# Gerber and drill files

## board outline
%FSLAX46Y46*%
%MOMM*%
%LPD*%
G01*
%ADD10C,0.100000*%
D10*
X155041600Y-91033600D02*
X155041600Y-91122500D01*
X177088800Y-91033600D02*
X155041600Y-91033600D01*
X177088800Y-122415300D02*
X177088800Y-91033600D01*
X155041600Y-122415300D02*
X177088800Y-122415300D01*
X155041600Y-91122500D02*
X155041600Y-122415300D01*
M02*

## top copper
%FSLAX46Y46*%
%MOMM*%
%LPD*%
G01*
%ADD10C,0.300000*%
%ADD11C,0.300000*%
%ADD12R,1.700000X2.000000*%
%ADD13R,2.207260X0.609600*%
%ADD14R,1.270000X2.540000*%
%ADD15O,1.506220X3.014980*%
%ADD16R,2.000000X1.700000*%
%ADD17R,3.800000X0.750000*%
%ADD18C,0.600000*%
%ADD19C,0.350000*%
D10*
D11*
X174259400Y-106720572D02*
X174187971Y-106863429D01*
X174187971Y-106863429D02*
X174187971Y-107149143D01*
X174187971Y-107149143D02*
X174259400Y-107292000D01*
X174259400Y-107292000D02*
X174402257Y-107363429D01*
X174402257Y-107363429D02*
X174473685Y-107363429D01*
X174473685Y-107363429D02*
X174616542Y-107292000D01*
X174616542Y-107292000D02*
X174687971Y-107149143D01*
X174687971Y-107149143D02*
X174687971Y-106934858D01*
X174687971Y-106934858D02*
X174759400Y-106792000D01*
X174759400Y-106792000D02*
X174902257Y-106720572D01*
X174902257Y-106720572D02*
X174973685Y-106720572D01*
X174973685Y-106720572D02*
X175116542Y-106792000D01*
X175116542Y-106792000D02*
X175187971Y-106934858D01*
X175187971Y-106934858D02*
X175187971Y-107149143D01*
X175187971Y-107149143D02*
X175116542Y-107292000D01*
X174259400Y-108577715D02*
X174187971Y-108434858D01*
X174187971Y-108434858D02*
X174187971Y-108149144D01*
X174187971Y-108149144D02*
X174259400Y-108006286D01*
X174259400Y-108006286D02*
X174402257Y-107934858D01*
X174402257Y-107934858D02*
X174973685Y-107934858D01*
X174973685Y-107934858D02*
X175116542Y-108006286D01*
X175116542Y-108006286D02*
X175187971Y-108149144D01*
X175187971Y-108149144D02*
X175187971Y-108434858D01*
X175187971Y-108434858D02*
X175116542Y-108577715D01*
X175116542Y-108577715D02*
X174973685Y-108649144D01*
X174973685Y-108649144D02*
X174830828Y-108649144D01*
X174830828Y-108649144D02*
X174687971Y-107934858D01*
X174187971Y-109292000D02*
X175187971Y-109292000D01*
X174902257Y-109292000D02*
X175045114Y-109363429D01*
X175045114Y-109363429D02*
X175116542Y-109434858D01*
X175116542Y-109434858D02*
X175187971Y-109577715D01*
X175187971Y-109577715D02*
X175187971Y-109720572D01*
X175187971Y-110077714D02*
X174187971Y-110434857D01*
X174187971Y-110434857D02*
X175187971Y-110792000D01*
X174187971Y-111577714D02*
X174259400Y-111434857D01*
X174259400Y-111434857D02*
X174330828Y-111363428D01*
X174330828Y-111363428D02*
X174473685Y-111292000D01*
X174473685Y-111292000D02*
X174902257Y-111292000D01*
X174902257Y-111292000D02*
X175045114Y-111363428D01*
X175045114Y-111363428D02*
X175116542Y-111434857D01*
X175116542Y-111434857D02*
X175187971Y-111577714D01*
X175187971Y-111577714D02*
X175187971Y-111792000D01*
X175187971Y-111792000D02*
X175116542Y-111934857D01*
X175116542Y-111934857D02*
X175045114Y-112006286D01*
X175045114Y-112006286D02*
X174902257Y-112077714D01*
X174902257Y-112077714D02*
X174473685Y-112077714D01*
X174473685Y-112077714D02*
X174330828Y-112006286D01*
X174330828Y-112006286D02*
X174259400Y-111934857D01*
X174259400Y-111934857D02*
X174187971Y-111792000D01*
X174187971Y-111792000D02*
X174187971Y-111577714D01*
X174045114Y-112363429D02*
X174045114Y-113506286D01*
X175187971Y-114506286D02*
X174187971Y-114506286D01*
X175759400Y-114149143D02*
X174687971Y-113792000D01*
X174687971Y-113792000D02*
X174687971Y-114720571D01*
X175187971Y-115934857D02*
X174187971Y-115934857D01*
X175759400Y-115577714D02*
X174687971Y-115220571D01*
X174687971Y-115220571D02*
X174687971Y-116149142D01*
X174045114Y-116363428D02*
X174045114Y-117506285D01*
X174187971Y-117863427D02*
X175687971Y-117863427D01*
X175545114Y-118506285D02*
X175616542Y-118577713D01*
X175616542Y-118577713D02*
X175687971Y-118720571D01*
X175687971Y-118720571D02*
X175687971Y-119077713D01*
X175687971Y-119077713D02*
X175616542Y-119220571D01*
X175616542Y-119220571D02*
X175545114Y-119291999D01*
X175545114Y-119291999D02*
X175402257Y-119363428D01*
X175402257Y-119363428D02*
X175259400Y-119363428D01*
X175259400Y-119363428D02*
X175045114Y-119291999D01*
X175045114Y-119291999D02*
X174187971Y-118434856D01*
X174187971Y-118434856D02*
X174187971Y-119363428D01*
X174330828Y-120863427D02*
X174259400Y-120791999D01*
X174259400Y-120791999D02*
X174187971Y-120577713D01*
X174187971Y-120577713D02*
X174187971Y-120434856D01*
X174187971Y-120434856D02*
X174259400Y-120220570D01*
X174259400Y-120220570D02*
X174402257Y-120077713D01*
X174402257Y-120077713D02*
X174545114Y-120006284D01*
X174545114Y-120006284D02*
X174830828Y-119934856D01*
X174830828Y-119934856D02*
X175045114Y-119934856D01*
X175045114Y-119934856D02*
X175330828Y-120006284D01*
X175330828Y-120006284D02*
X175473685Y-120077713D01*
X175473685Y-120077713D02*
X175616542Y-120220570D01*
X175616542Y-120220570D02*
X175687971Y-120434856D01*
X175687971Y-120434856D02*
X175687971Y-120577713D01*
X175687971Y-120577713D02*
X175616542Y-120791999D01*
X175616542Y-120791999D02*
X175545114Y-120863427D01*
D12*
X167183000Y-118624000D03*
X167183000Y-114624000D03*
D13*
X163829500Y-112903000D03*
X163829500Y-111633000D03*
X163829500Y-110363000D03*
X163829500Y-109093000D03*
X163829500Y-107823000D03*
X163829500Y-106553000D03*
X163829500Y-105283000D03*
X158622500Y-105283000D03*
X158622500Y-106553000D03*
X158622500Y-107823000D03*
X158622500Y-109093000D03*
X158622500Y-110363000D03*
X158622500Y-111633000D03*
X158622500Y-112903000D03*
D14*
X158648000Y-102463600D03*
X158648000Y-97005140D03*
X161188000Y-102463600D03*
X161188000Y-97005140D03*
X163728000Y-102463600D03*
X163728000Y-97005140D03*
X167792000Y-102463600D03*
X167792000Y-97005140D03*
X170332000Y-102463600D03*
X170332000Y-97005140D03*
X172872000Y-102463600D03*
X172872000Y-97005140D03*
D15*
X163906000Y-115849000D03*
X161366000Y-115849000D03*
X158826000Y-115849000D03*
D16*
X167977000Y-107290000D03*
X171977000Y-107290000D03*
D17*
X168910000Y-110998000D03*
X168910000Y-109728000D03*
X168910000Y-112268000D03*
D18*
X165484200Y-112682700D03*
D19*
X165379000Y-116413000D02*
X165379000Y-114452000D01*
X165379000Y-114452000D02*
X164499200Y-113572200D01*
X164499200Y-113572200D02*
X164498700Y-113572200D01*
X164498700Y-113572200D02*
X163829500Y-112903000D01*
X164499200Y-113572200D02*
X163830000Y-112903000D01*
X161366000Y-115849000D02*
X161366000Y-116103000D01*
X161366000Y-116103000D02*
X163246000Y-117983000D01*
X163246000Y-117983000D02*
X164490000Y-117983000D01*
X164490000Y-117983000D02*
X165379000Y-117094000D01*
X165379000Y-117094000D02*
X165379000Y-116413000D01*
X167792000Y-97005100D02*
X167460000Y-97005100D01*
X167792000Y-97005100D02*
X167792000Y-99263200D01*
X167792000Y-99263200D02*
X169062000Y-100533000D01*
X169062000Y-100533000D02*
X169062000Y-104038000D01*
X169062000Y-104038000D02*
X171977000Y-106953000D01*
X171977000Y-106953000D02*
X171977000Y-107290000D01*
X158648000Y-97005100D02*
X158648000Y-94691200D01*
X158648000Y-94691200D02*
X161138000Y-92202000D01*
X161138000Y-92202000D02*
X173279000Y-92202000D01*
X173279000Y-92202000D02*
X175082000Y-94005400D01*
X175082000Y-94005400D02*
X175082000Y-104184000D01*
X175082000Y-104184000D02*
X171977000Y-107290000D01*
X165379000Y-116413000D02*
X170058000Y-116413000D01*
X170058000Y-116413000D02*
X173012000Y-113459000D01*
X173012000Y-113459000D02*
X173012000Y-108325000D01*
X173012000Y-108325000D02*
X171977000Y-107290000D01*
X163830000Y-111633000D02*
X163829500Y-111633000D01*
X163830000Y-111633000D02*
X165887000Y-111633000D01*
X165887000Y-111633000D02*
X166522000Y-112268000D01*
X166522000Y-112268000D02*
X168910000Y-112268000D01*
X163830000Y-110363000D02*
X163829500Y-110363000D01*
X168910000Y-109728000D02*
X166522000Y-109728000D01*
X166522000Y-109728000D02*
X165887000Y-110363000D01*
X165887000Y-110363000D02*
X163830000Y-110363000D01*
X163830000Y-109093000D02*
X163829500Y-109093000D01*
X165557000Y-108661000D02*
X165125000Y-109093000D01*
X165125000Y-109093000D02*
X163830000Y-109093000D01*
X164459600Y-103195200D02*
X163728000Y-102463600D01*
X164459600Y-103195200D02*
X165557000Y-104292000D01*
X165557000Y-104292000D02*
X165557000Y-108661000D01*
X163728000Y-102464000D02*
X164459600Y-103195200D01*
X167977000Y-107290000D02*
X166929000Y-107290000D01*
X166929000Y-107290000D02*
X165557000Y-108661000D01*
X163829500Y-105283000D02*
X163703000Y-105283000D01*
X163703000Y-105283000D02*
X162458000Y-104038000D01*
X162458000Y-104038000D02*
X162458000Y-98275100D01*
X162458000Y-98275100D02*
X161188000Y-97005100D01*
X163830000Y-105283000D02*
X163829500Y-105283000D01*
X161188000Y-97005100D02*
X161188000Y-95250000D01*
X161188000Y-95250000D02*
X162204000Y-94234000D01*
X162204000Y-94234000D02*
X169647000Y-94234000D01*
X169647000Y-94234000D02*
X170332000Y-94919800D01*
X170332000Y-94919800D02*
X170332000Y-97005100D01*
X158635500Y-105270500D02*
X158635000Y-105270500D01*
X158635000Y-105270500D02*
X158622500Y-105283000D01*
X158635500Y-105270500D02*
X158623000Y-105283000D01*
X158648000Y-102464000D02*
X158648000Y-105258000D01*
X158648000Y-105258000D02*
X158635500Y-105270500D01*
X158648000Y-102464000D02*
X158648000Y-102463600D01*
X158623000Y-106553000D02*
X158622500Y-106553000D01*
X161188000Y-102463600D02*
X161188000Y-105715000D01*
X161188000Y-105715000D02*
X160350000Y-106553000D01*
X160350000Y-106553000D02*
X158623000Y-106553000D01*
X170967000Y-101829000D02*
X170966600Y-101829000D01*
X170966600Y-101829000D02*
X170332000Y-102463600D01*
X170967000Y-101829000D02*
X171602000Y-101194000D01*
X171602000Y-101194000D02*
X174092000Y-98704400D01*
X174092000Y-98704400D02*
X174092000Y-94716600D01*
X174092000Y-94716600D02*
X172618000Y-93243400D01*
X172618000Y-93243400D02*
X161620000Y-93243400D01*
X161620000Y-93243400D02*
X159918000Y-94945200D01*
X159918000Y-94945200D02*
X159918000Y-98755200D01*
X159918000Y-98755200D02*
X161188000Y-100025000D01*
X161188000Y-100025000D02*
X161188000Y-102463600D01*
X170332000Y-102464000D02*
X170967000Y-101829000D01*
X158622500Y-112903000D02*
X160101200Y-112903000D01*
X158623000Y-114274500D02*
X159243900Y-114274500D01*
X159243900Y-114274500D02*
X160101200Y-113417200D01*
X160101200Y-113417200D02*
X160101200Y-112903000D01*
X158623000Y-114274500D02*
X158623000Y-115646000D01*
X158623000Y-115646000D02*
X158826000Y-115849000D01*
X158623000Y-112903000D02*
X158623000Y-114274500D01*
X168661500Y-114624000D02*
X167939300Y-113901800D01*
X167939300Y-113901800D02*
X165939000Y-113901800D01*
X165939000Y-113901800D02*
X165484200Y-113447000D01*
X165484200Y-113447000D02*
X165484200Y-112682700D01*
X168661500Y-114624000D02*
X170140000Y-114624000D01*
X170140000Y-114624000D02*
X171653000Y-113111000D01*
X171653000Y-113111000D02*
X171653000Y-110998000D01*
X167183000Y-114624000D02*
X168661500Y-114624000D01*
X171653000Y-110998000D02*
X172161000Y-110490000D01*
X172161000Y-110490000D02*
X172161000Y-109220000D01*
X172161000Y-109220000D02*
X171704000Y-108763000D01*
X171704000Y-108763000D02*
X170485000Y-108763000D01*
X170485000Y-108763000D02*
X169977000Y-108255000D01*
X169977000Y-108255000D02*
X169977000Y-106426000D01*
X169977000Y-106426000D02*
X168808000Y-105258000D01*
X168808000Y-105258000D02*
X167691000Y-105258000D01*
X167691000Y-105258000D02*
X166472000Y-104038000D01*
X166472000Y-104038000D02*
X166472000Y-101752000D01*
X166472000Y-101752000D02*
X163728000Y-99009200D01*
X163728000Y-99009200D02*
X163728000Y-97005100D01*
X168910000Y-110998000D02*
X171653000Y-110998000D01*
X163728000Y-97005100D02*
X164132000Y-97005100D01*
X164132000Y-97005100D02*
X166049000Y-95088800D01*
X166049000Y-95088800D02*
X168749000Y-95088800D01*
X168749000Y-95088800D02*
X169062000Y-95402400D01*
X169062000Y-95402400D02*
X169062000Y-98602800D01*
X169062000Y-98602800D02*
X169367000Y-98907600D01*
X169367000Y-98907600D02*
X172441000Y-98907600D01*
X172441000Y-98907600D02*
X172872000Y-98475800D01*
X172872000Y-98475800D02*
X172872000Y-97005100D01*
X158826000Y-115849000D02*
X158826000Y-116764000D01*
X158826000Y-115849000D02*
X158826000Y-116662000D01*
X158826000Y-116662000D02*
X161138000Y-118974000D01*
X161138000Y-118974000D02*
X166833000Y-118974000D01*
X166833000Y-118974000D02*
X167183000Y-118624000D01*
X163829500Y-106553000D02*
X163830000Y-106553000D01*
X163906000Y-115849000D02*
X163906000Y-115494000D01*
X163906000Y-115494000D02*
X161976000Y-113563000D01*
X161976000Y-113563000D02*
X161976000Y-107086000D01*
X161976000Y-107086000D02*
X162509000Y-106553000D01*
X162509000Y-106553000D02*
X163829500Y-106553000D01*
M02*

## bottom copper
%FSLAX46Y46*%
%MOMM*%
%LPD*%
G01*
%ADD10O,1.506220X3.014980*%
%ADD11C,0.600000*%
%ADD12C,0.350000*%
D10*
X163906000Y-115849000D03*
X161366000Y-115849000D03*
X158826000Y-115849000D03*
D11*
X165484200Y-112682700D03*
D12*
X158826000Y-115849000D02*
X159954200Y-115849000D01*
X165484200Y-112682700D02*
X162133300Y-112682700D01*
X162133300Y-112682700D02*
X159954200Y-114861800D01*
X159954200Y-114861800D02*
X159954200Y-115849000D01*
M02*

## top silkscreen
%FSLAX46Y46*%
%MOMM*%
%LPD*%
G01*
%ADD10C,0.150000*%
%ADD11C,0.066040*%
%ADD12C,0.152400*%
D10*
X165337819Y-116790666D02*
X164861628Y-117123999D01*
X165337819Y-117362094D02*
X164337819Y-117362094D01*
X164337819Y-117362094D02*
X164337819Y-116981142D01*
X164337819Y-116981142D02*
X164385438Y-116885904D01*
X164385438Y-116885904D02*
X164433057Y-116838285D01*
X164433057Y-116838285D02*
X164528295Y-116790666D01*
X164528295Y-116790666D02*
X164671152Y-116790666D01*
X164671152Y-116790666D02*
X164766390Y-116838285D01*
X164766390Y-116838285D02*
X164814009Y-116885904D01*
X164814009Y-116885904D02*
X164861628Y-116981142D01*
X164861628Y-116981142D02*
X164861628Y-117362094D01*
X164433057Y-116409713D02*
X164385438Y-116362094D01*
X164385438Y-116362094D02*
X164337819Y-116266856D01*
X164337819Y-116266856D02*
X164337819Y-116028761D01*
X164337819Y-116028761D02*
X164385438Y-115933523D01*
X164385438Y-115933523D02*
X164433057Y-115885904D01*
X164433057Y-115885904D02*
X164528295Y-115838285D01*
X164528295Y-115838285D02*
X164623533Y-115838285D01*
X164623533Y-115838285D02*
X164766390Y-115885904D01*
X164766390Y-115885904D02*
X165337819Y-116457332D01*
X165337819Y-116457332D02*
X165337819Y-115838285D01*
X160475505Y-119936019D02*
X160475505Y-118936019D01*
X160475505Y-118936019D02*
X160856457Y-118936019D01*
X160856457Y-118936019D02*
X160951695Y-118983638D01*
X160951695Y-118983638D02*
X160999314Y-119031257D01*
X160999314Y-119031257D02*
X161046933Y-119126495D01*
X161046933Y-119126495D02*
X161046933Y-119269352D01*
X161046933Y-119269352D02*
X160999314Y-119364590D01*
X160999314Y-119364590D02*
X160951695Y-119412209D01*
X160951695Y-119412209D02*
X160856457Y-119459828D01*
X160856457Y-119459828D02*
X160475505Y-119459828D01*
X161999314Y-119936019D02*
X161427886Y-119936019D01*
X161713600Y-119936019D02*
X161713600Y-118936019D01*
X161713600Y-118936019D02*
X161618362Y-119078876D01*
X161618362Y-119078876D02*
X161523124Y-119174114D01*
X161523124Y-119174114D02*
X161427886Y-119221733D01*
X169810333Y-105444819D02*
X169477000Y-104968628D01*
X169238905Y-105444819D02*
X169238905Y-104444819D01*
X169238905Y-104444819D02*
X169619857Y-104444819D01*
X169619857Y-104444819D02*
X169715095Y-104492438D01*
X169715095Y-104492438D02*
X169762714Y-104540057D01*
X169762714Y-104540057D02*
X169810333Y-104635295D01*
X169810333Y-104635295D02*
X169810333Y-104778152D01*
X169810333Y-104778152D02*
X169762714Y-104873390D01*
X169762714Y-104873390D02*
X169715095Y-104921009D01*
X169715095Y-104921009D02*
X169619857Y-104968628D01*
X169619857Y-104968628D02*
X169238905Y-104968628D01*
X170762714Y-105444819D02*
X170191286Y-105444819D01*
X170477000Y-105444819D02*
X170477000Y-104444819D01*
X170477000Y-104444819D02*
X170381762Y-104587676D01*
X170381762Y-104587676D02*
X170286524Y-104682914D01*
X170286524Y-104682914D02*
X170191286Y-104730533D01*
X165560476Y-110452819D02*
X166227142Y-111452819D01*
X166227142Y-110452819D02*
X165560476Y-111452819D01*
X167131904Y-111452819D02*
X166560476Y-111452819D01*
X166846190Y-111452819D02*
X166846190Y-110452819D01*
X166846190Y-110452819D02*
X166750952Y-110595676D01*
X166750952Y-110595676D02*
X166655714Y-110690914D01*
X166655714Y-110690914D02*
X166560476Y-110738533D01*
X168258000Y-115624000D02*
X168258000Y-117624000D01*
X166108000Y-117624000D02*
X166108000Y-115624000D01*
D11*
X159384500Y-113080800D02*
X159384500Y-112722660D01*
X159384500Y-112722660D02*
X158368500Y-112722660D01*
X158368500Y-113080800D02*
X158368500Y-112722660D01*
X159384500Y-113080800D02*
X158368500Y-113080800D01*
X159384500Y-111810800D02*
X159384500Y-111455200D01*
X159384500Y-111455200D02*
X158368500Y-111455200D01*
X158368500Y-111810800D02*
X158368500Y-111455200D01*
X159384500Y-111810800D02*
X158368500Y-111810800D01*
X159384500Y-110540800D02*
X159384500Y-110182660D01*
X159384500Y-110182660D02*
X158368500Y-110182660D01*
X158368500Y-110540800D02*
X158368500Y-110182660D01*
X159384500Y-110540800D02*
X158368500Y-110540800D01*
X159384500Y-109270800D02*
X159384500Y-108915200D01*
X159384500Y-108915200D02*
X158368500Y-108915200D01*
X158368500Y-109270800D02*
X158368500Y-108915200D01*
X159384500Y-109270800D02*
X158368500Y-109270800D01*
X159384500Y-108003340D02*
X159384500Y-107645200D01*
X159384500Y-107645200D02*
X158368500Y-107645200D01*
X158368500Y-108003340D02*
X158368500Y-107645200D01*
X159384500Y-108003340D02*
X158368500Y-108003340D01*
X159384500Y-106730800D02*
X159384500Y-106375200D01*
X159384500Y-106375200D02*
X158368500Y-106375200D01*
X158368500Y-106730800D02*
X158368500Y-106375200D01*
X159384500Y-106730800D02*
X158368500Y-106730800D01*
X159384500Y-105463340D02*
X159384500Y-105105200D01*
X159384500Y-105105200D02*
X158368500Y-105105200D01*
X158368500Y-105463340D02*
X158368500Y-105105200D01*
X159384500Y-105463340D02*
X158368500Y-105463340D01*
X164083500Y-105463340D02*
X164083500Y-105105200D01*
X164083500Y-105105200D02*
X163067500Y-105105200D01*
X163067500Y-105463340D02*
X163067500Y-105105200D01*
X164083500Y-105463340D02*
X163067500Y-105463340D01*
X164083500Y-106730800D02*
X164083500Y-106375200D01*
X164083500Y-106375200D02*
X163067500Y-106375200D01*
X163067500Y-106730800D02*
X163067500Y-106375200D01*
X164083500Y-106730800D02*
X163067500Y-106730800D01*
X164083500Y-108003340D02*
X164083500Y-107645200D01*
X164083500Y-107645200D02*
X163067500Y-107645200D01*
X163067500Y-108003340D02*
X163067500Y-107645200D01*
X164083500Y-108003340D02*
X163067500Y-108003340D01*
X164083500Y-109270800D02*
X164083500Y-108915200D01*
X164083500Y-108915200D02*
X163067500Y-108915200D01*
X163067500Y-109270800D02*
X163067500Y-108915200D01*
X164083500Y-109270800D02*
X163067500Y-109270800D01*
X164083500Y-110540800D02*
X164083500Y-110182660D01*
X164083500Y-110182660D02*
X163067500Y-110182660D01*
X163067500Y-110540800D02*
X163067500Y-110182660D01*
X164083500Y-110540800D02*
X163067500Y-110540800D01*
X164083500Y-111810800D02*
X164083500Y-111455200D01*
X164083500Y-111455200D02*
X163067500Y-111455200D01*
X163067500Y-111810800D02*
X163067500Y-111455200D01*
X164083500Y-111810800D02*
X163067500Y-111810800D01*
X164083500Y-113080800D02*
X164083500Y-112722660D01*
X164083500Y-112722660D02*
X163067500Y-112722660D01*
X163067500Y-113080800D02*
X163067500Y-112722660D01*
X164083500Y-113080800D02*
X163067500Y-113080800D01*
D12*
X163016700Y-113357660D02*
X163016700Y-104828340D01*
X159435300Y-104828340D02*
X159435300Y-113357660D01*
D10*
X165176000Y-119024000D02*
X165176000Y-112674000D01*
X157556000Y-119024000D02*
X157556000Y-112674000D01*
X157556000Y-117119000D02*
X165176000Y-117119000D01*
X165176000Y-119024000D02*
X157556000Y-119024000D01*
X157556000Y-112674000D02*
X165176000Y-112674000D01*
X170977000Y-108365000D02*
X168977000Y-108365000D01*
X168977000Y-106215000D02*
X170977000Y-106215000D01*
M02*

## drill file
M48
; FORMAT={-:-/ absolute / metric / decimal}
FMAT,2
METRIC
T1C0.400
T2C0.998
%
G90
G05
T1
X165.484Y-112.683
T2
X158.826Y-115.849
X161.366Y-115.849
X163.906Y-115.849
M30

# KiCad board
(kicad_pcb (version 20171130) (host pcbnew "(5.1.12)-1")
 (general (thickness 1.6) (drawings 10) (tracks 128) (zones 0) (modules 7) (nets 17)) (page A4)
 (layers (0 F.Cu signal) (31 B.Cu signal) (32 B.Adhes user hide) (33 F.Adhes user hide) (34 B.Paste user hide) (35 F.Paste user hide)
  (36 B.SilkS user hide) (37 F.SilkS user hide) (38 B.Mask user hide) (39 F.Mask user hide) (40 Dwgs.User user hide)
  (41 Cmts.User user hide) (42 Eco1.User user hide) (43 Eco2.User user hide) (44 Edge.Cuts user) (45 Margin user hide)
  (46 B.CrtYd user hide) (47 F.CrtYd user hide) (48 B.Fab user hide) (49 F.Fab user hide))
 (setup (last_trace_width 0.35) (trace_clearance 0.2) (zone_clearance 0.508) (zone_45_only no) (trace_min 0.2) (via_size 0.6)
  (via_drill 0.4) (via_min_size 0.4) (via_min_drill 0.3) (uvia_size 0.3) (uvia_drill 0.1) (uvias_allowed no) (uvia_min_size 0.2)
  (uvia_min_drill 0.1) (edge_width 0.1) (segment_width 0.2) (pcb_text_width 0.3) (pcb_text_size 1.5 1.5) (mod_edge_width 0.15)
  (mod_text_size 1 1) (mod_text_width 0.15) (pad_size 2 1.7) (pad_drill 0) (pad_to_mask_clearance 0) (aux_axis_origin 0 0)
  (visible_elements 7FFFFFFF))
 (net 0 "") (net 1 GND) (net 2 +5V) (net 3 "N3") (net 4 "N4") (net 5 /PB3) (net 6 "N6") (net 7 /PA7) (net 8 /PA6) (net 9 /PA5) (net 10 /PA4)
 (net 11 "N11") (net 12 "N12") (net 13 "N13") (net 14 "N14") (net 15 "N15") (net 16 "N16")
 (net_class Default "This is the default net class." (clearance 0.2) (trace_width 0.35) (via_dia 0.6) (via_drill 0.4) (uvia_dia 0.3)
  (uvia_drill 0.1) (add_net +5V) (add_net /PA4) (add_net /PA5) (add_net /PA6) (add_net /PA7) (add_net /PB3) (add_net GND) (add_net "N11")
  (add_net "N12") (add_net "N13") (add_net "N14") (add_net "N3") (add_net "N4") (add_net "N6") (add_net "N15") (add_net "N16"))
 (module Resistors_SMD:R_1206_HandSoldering (layer F.Cu) (at 167.183 116.624 90)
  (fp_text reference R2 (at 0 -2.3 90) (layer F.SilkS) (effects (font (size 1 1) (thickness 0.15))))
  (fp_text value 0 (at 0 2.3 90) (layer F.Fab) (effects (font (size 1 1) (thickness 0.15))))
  (fp_line (start 1 1.075) (end -1 1.075) (layer F.SilkS) (width 0.15))
  (fp_line (start -1 -1.075) (end 1 -1.075) (layer F.SilkS) (width 0.15))
  (pad 2 smd rect (at -2 0 90) (size 2 1.7) (layers F.Cu F.Paste F.Mask) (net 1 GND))
  (pad 1 smd rect (at 2 0 90) (size 2 1.7) (layers F.Cu F.Paste F.Mask) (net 1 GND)))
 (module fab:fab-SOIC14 (layer F.Cu) (at 161.226 109.093 90)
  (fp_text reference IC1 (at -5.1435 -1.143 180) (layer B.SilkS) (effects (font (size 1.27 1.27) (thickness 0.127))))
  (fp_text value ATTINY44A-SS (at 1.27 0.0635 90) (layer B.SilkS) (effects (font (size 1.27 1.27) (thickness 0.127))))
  (fp_line (start -3.9878 -1.8415) (end -3.62966 -1.8415) (layer F.SilkS) (width 0.06604))
  (fp_line (start -3.62966 -1.8415) (end -3.62966 -2.8575) (layer F.SilkS) (width 0.06604))
  (fp_line (start -3.9878 -2.8575) (end -3.62966 -2.8575) (layer F.SilkS) (width 0.06604))
  (fp_line (start -3.9878 -1.8415) (end -3.9878 -2.8575) (layer F.SilkS) (width 0.06604))
  (fp_line (start -2.7178 -1.8415) (end -2.3622 -1.8415) (layer F.SilkS) (width 0.06604))
  (fp_line (start -2.3622 -1.8415) (end -2.3622 -2.8575) (layer F.SilkS) (width 0.06604))
  (fp_line (start -2.7178 -2.8575) (end -2.3622 -2.8575) (layer F.SilkS) (width 0.06604))
  (fp_line (start -2.7178 -1.8415) (end -2.7178 -2.8575) (layer F.SilkS) (width 0.06604))
  (fp_line (start -1.4478 -1.8415) (end -1.08966 -1.8415) (layer F.SilkS) (width 0.06604))
  (fp_line (start -1.08966 -1.8415) (end -1.08966 -2.8575) (layer F.SilkS) (width 0.06604))
  (fp_line (start -1.4478 -2.8575) (end -1.08966 -2.8575) (layer F.SilkS) (width 0.06604))
  (fp_line (start -1.4478 -1.8415) (end -1.4478 -2.8575) (layer F.SilkS) (width 0.06604))
  (fp_line (start -0.1778 -1.8415) (end 0.1778 -1.8415) (layer F.SilkS) (width 0.06604))
  (fp_line (start 0.1778 -1.8415) (end 0.1778 -2.8575) (layer F.SilkS) (width 0.06604))
  (fp_line (start -0.1778 -2.8575) (end 0.1778 -2.8575) (layer F.SilkS) (width 0.06604))
  (fp_line (start -0.1778 -1.8415) (end -0.1778 -2.8575) (layer F.SilkS) (width 0.06604))
  (fp_line (start 1.08966 -1.8415) (end 1.4478 -1.8415) (layer F.SilkS) (width 0.06604))
  (fp_line (start 1.4478 -1.8415) (end 1.4478 -2.8575) (layer F.SilkS) (width 0.06604))
  (fp_line (start 1.08966 -2.8575) (end 1.4478 -2.8575) (layer F.SilkS) (width 0.06604))
  (fp_line (start 1.08966 -1.8415) (end 1.08966 -2.8575) (layer F.SilkS) (width 0.06604))
  (fp_line (start 2.3622 -1.8415) (end 2.7178 -1.8415) (layer F.SilkS) (width 0.06604))
  (fp_line (start 2.7178 -1.8415) (end 2.7178 -2.8575) (layer F.SilkS) (width 0.06604))
  (fp_line (start 2.3622 -2.8575) (end 2.7178 -2.8575) (layer F.SilkS) (width 0.06604))
  (fp_line (start 2.3622 -1.8415) (end 2.3622 -2.8575) (layer F.SilkS) (width 0.06604))
  (fp_line (start 3.62966 -1.8415) (end 3.9878 -1.8415) (layer F.SilkS) (width 0.06604))
  (fp_line (start 3.9878 -1.8415) (end 3.9878 -2.8575) (layer F.SilkS) (width 0.06604))
  (fp_line (start 3.62966 -2.8575) (end 3.9878 -2.8575) (layer F.SilkS) (width 0.06604))
  (fp_line (start 3.62966 -1.8415) (end 3.62966 -2.8575) (layer F.SilkS) (width 0.06604))
  (fp_line (start 3.62966 2.8575) (end 3.9878 2.8575) (layer F.SilkS) (width 0.06604))
  (fp_line (start 3.9878 2.8575) (end 3.9878 1.8415) (layer F.SilkS) (width 0.06604))
  (fp_line (start 3.62966 1.8415) (end 3.9878 1.8415) (layer F.SilkS) (width 0.06604))
  (fp_line (start 3.62966 2.8575) (end 3.62966 1.8415) (layer F.SilkS) (width 0.06604))
  (fp_line (start 2.3622 2.8575) (end 2.7178 2.8575) (layer F.SilkS) (width 0.06604))
  (fp_line (start 2.7178 2.8575) (end 2.7178 1.8415) (layer F.SilkS) (width 0.06604))
  (fp_line (start 2.3622 1.8415) (end 2.7178 1.8415) (layer F.SilkS) (width 0.06604))
  (fp_line (start 2.3622 2.8575) (end 2.3622 1.8415) (layer F.SilkS) (width 0.06604))
  (fp_line (start 1.08966 2.8575) (end 1.4478 2.8575) (layer F.SilkS) (width 0.06604))
  (fp_line (start 1.4478 2.8575) (end 1.4478 1.8415) (layer F.SilkS) (width 0.06604))
  (fp_line (start 1.08966 1.8415) (end 1.4478 1.8415) (layer F.SilkS) (width 0.06604))
  (fp_line (start 1.08966 2.8575) (end 1.08966 1.8415) (layer F.SilkS) (width 0.06604))
  (fp_line (start -0.1778 2.8575) (end 0.1778 2.8575) (layer F.SilkS) (width 0.06604))
  (fp_line (start 0.1778 2.8575) (end 0.1778 1.8415) (layer F.SilkS) (width 0.06604))
  (fp_line (start -0.1778 1.8415) (end 0.1778 1.8415) (layer F.SilkS) (width 0.06604))
  (fp_line (start -0.1778 2.8575) (end -0.1778 1.8415) (layer F.SilkS) (width 0.06604))
  (fp_line (start -1.4478 2.8575) (end -1.08966 2.8575) (layer F.SilkS) (width 0.06604))
  (fp_line (start -1.08966 2.8575) (end -1.08966 1.8415) (layer F.SilkS) (width 0.06604))
  (fp_line (start -1.4478 1.8415) (end -1.08966 1.8415) (layer F.SilkS) (width 0.06604))
  (fp_line (start -1.4478 2.8575) (end -1.4478 1.8415) (layer F.SilkS) (width 0.06604))
  (fp_line (start -2.7178 2.8575) (end -2.3622 2.8575) (layer F.SilkS) (width 0.06604))
  (fp_line (start -2.3622 2.8575) (end -2.3622 1.8415) (layer F.SilkS) (width 0.06604))
  (fp_line (start -2.7178 1.8415) (end -2.3622 1.8415) (layer F.SilkS) (width 0.06604))
  (fp_line (start -2.7178 2.8575) (end -2.7178 1.8415) (layer F.SilkS) (width 0.06604))
  (fp_line (start -3.9878 2.8575) (end -3.62966 2.8575) (layer F.SilkS) (width 0.06604))
  (fp_line (start -3.62966 2.8575) (end -3.62966 1.8415) (layer F.SilkS) (width 0.06604))
  (fp_line (start -3.9878 1.8415) (end -3.62966 1.8415) (layer F.SilkS) (width 0.06604))
  (fp_line (start -3.9878 2.8575) (end -3.9878 1.8415) (layer F.SilkS) (width 0.06604))
  (fp_line (start -4.26466 1.7907) (end 4.26466 1.7907) (layer F.SilkS) (width 0.1524))
  (fp_line (start 4.26466 -1.7907) (end -4.26466 -1.7907) (layer F.SilkS) (width 0.1524))
  (pad 1 smd rect (at -3.81 2.6035 90) (size 0.6096 2.20726) (layers F.Cu F.Paste F.Mask) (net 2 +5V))
  (pad 2 smd rect (at -2.54 2.6035 90) (size 0.6096 2.20726) (layers F.Cu F.Paste F.Mask) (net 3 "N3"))
  (pad 3 smd rect (at -1.27 2.6035 90) (size 0.6096 2.20726) (layers F.Cu F.Paste F.Mask) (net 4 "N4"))
  (pad 4 smd rect (at 0 2.6035 90) (size 0.6096 2.20726) (layers F.Cu F.Paste F.Mask) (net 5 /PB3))
  (pad 5 smd rect (at 1.27 2.6035 90) (size 0.6096 2.20726) (layers F.Cu F.Paste F.Mask) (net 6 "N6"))
  (pad 6 smd rect (at 2.54 2.6035 90) (size 0.6096 2.20726) (layers F.Cu F.Paste F.Mask) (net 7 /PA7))
  (pad 7 smd rect (at 3.81 2.6035 90) (size 0.6096 2.20726) (layers F.Cu F.Paste F.Mask) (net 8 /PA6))
  (pad 8 smd rect (at 3.81 -2.6035 90) (size 0.6096 2.20726) (layers F.Cu F.Paste F.Mask) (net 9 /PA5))
  (pad 9 smd rect (at 2.54 -2.6035 90) (size 0.6096 2.20726) (layers F.Cu F.Paste F.Mask) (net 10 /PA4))
  (pad 10 smd rect (at 1.27 -2.6035 90) (size 0.6096 2.20726) (layers F.Cu F.Paste F.Mask) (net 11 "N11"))
  (pad 11 smd rect (at 0 -2.6035 90) (size 0.6096 2.20726) (layers F.Cu F.Paste F.Mask) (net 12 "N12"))
  (pad 12 smd rect (at -1.27 -2.6035 90) (size 0.6096 2.20726) (layers F.Cu F.Paste F.Mask) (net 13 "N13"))
  (pad 13 smd rect (at -2.54 -2.6035 90) (size 0.6096 2.20726) (layers F.Cu F.Paste F.Mask) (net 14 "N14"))
  (pad 14 smd rect (at -3.81 -2.6035 90) (size 0.6096 2.20726) (layers F.Cu F.Paste F.Mask) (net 1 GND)))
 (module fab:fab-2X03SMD (layer F.Cu) (at 161.188 99.9236 90)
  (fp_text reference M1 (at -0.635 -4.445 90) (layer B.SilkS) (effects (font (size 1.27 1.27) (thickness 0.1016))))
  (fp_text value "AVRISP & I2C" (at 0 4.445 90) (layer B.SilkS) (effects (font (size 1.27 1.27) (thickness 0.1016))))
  (pad 1 smd rect (at -2.54 -2.54 90) (size 2.54 1.27) (layers F.Cu F.Paste F.Mask) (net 9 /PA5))
  (pad 2 smd rect (at 2.91846 -2.54 90) (size 2.54 1.27) (layers F.Cu F.Paste F.Mask) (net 2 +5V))
  (pad 3 smd rect (at -2.54 0 90) (size 2.54 1.27) (layers F.Cu F.Paste F.Mask) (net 10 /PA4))
  (pad 4 smd rect (at 2.91846 0 90) (size 2.54 1.27) (layers F.Cu F.Paste F.Mask) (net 8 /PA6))
  (pad 5 smd rect (at -2.54 2.54 90) (size 2.54 1.27) (layers F.Cu F.Paste F.Mask) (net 5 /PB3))
  (pad 6 smd rect (at 2.91846 2.54 90) (size 2.54 1.27) (layers F.Cu F.Paste F.Mask) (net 1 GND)))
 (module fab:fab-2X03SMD (layer F.Cu) (at 170.332 99.9236 90)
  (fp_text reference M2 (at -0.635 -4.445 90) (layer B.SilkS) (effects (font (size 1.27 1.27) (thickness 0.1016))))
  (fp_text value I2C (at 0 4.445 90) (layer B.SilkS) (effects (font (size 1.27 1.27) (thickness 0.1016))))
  (pad 1 smd rect (at -2.54 -2.54 90) (size 2.54 1.27) (layers F.Cu F.Paste F.Mask) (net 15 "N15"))
  (pad 2 smd rect (at 2.91846 -2.54 90) (size 2.54 1.27) (layers F.Cu F.Paste F.Mask) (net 2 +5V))
  (pad 3 smd rect (at -2.54 0 90) (size 2.54 1.27) (layers F.Cu F.Paste F.Mask) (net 10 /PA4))
  (pad 4 smd rect (at 2.91846 0 90) (size 2.54 1.27) (layers F.Cu F.Paste F.Mask) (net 8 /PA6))
  (pad 5 smd rect (at -2.54 2.54 90) (size 2.54 1.27) (layers F.Cu F.Paste F.Mask) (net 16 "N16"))
  (pad 6 smd rect (at 2.91846 2.54 90) (size 2.54 1.27) (layers F.Cu F.Paste F.Mask) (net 1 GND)))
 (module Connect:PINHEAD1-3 (layer F.Cu) (at 161.366 115.849 180)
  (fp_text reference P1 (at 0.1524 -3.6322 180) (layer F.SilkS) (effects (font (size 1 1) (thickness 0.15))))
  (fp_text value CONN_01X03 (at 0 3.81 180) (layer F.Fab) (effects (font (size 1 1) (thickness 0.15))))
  (fp_line (start -3.81 -3.175) (end -3.81 3.175) (layer F.SilkS) (width 0.15))
  (fp_line (start 3.81 -3.175) (end 3.81 3.175) (layer F.SilkS) (width 0.15))
  (fp_line (start 3.81 -1.27) (end -3.81 -1.27) (layer F.SilkS) (width 0.15))
  (fp_line (start -3.81 -3.175) (end 3.81 -3.175) (layer F.SilkS) (width 0.15))
  (fp_line (start 3.81 3.175) (end -3.81 3.175) (layer F.SilkS) (width 0.15))
  (pad 1 thru_hole oval (at -2.54 0 180) (size 1.50622 3.01498) (drill 0.99822) (layers *.Cu *.Mask) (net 7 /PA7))
  (pad 2 thru_hole oval (at 0 0 180) (size 1.50622 3.01498) (drill 0.99822) (layers *.Cu *.Mask) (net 2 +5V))
  (pad 3 thru_hole oval (at 2.54 0 180) (size 1.50622 3.01498) (drill 0.99822) (layers *.Cu *.Mask) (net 1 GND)))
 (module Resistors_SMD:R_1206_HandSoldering (layer F.Cu) (at 169.977 107.29)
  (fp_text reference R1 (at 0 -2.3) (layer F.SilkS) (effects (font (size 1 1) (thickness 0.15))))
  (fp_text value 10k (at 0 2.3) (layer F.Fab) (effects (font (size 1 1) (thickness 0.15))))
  (fp_line (start 1 1.075) (end -1 1.075) (layer F.SilkS) (width 0.15))
  (fp_line (start -1 -1.075) (end 1 -1.075) (layer F.SilkS) (width 0.15))
  (pad 1 smd rect (at -2 0) (size 2 1.7) (layers F.Cu F.Paste F.Mask) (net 5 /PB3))
  (pad 2 smd rect (at 2 0) (size 2 1.7) (layers F.Cu F.Paste F.Mask) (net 2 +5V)))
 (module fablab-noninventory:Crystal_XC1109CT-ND (layer F.Cu) (at 168.91 110.998 90)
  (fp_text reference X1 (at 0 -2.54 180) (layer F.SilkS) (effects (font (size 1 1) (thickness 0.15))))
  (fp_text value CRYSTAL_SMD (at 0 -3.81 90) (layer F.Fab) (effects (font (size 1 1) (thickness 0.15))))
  (pad 2 smd rect (at 0 0 90) (size 0.75 3.8) (layers F.Cu F.Paste F.Mask) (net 1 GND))
  (pad 1 smd rect (at 1.27 0 90) (size 0.75 3.8) (layers F.Cu F.Paste F.Mask) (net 4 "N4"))
  (pad 3 smd rect (at -1.27 0 90) (size 0.75 3.8) (layers F.Cu F.Paste F.Mask) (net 3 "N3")))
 (gr_line (start 155.0416 91.0336) (end 155.0416 91.1225) (angle 90) (layer Edge.Cuts) (width 0.1))
 (gr_line (start 177.0888 91.0336) (end 155.0416 91.0336) (angle 90) (layer Edge.Cuts) (width 0.1))
 (gr_line (start 177.0888 122.4153) (end 177.0888 91.0336) (angle 90) (layer Edge.Cuts) (width 0.1))
 (gr_line (start 155.0416 122.4153) (end 177.0888 122.4153) (angle 90) (layer Edge.Cuts) (width 0.1))
 (gr_line (start 155.0416 91.1225) (end 155.0416 122.4153) (angle 90) (layer Edge.Cuts) (width 0.1))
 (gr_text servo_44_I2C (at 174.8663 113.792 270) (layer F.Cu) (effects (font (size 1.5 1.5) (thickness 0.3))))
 (segment (start 165.379 116.413) (end 165.379 114.452) (width 0.35) (layer F.Cu) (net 2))
 (segment (start 165.379 114.452) (end 164.4992 113.5722) (width 0.35) (layer F.Cu) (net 2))
 (segment (start 164.4992 113.5722) (end 164.4987 113.5722) (width 0.35) (layer F.Cu) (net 2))
 (segment (start 164.4987 113.5722) (end 163.8295 112.903) (width 0.35) (layer F.Cu) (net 2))
 (segment (start 164.4992 113.5722) (end 163.83 112.903) (width 0.35) (layer F.Cu) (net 2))
 (segment (start 161.366 115.849) (end 161.366 116.103) (width 0.35) (layer F.Cu) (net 2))
 (segment (start 161.366 116.103) (end 163.246 117.983) (width 0.35) (layer F.Cu) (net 2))
 (segment (start 163.246 117.983) (end 164.49 117.983) (width 0.35) (layer F.Cu) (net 2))
 (segment (start 164.49 117.983) (end 165.379 117.094) (width 0.35) (layer F.Cu) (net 2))
 (segment (start 165.379 117.094) (end 165.379 116.413) (width 0.35) (layer F.Cu) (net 2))
 (segment (start 167.792 97.0051) (end 167.46 97.0051) (width 0.35) (layer F.Cu) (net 2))
 (segment (start 167.792 97.0051) (end 167.792 99.2632) (width 0.35) (layer F.Cu) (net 2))
 (segment (start 167.792 99.2632) (end 169.062 100.533) (width 0.35) (layer F.Cu) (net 2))
 (segment (start 169.062 100.533) (end 169.062 104.038) (width 0.35) (layer F.Cu) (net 2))
 (segment (start 169.062 104.038) (end 171.977 106.953) (width 0.35) (layer F.Cu) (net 2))
 (segment (start 171.977 106.953) (end 171.977 107.29) (width 0.35) (layer F.Cu) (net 2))
 (segment (start 158.648 97.0051) (end 158.648 94.6912) (width 0.35) (layer F.Cu) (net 2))
 (segment (start 158.648 94.6912) (end 161.138 92.202) (width 0.35) (layer F.Cu) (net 2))
 (segment (start 161.138 92.202) (end 173.279 92.202) (width 0.35) (layer F.Cu) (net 2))
 (segment (start 173.279 92.202) (end 175.082 94.0054) (width 0.35) (layer F.Cu) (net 2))
 (segment (start 175.082 94.0054) (end 175.082 104.184) (width 0.35) (layer F.Cu) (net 2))
 (segment (start 175.082 104.184) (end 171.977 107.29) (width 0.35) (layer F.Cu) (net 2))
 (segment (start 165.379 116.413) (end 170.058 116.413) (width 0.35) (layer F.Cu) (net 2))
 (segment (start 170.058 116.413) (end 173.012 113.459) (width 0.35) (layer F.Cu) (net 2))
 (segment (start 173.012 113.459) (end 173.012 108.325) (width 0.35) (layer F.Cu) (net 2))
 (segment (start 173.012 108.325) (end 171.977 107.29) (width 0.35) (layer F.Cu) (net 2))
 (segment (start 163.83 111.633) (end 163.8295 111.633) (width 0.35) (layer F.Cu) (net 3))
 (segment (start 163.83 111.633) (end 165.887 111.633) (width 0.35) (layer F.Cu) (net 3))
 (segment (start 165.887 111.633) (end 166.522 112.268) (width 0.35) (layer F.Cu) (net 3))
 (segment (start 166.522 112.268) (end 168.91 112.268) (width 0.35) (layer F.Cu) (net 3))
 (segment (start 163.83 110.363) (end 163.8295 110.363) (width 0.35) (layer F.Cu) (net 4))
 (segment (start 168.91 109.728) (end 166.522 109.728) (width 0.35) (layer F.Cu) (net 4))
 (segment (start 166.522 109.728) (end 165.887 110.363) (width 0.35) (layer F.Cu) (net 4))
 (segment (start 165.887 110.363) (end 163.83 110.363) (width 0.35) (layer F.Cu) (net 4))
 (segment (start 163.83 109.093) (end 163.8295 109.093) (width 0.35) (layer F.Cu) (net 5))
 (segment (start 165.557 108.661) (end 165.125 109.093) (width 0.35) (layer F.Cu) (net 5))
 (segment (start 165.125 109.093) (end 163.83 109.093) (width 0.35) (layer F.Cu) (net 5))
 (segment (start 164.4596 103.1952) (end 163.728 102.4636) (width 0.35) (layer F.Cu) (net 5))
 (segment (start 164.4596 103.1952) (end 165.557 104.292) (width 0.35) (layer F.Cu) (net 5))
 (segment (start 165.557 104.292) (end 165.557 108.661) (width 0.35) (layer F.Cu) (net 5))
 (segment (start 163.728 102.464) (end 164.4596 103.1952) (width 0.35) (layer F.Cu) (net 5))
 (segment (start 167.977 107.29) (end 166.929 107.29) (width 0.35) (layer F.Cu) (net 5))
 (segment (start 166.929 107.29) (end 165.557 108.661) (width 0.35) (layer F.Cu) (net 5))
 (segment (start 163.8295 105.283) (end 163.703 105.283) (width 0.35) (layer F.Cu) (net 8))
 (segment (start 163.703 105.283) (end 162.458 104.038) (width 0.35) (layer F.Cu) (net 8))
 (segment (start 162.458 104.038) (end 162.458 98.2751) (width 0.35) (layer F.Cu) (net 8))
 (segment (start 162.458 98.2751) (end 161.188 97.0051) (width 0.35) (layer F.Cu) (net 8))
 (segment (start 163.83 105.283) (end 163.8295 105.283) (width 0.35) (layer F.Cu) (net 8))
 (segment (start 161.188 97.0051) (end 161.188 95.25) (width 0.35) (layer F.Cu) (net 8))
 (segment (start 161.188 95.25) (end 162.204 94.234) (width 0.35) (layer F.Cu) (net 8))
 (segment (start 162.204 94.234) (end 169.647 94.234) (width 0.35) (layer F.Cu) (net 8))
 (segment (start 169.647 94.234) (end 170.332 94.9198) (width 0.35) (layer F.Cu) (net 8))
 (segment (start 170.332 94.9198) (end 170.332 97.0051) (width 0.35) (layer F.Cu) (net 8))
 (segment (start 158.6355 105.2705) (end 158.635 105.2705) (width 0.35) (layer F.Cu) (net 9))
 (segment (start 158.635 105.2705) (end 158.6225 105.283) (width 0.35) (layer F.Cu) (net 9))
 (segment (start 158.6355 105.2705) (end 158.623 105.283) (width 0.35) (layer F.Cu) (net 9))
 (segment (start 158.648 102.464) (end 158.648 105.258) (width 0.35) (layer F.Cu) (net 9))
 (segment (start 158.648 105.258) (end 158.6355 105.2705) (width 0.35) (layer F.Cu) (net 9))
 (segment (start 158.648 102.464) (end 158.648 102.4636) (width 0.35) (layer F.Cu) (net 9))
 (segment (start 158.623 106.553) (end 158.6225 106.553) (width 0.35) (layer F.Cu) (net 10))
 (segment (start 161.188 102.4636) (end 161.188 105.715) (width 0.35) (layer F.Cu) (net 10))
 (segment (start 161.188 105.715) (end 160.35 106.553) (width 0.35) (layer F.Cu) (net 10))
 (segment (start 160.35 106.553) (end 158.623 106.553) (width 0.35) (layer F.Cu) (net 10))
 (segment (start 170.967 101.829) (end 170.9666 101.829) (width 0.35) (layer F.Cu) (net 10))
 (segment (start 170.9666 101.829) (end 170.332 102.4636) (width 0.35) (layer F.Cu) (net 10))
 (segment (start 170.967 101.829) (end 171.602 101.194) (width 0.35) (layer F.Cu) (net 10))
 (segment (start 171.602 101.194) (end 174.092 98.7044) (width 0.35) (layer F.Cu) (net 10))
 (segment (start 174.092 98.7044) (end 174.092 94.7166) (width 0.35) (layer F.Cu) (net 10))
 (segment (start 174.092 94.7166) (end 172.618 93.2434) (width 0.35) (layer F.Cu) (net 10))
 (segment (start 172.618 93.2434) (end 161.62 93.2434) (width 0.35) (layer F.Cu) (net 10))
 (segment (start 161.62 93.2434) (end 159.918 94.9452) (width 0.35) (layer F.Cu) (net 10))
 (segment (start 159.918 94.9452) (end 159.918 98.7552) (width 0.35) (layer F.Cu) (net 10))
 (segment (start 159.918 98.7552) (end 161.188 100.025) (width 0.35) (layer F.Cu) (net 10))
 (segment (start 161.188 100.025) (end 161.188 102.4636) (width 0.35) (layer F.Cu) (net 10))
 (segment (start 170.332 102.464) (end 170.967 101.829) (width 0.35) (layer F.Cu) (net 10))
 (segment (start 158.6225 112.903) (end 160.1012 112.903) (width 0.35) (layer F.Cu) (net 1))
 (segment (start 158.623 114.2745) (end 159.2439 114.2745) (width 0.35) (layer F.Cu) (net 1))
 (segment (start 159.2439 114.2745) (end 160.1012 113.4172) (width 0.35) (layer F.Cu) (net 1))
 (segment (start 160.1012 113.4172) (end 160.1012 112.903) (width 0.35) (layer F.Cu) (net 1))
 (segment (start 158.623 114.2745) (end 158.623 115.646) (width 0.35) (layer F.Cu) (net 1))
 (segment (start 158.623 115.646) (end 158.826 115.849) (width 0.35) (layer F.Cu) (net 1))
 (segment (start 158.623 112.903) (end 158.623 114.2745) (width 0.35) (layer F.Cu) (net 1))
 (segment (start 158.826 115.849) (end 159.9542 115.849) (width 0.35) (layer B.Cu) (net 1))
 (segment (start 165.4842 112.6827) (end 162.1333 112.6827) (width 0.35) (layer B.Cu) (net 1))
 (segment (start 162.1333 112.6827) (end 159.9542 114.8618) (width 0.35) (layer B.Cu) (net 1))
 (segment (start 159.9542 114.8618) (end 159.9542 115.849) (width 0.35) (layer B.Cu) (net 1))
 (segment (start 168.6615 114.624) (end 167.9393 113.9018) (width 0.35) (layer F.Cu) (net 1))
 (segment (start 167.9393 113.9018) (end 165.939 113.9018) (width 0.35) (layer F.Cu) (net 1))
 (segment (start 165.939 113.9018) (end 165.4842 113.447) (width 0.35) (layer F.Cu) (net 1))
 (segment (start 165.4842 113.447) (end 165.4842 112.6827) (width 0.35) (layer F.Cu) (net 1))
 (segment (start 168.6615 114.624) (end 170.14 114.624) (width 0.35) (layer F.Cu) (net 1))
 (segment (start 170.14 114.624) (end 171.653 113.111) (width 0.35) (layer F.Cu) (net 1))
 (segment (start 171.653 113.111) (end 171.653 110.998) (width 0.35) (layer F.Cu) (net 1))
 (segment (start 167.183 114.624) (end 168.6615 114.624) (width 0.35) (layer F.Cu) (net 1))
 (segment (start 171.653 110.998) (end 172.161 110.49) (width 0.35) (layer F.Cu) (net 1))
 (segment (start 172.161 110.49) (end 172.161 109.22) (width 0.35) (layer F.Cu) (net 1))
 (segment (start 172.161 109.22) (end 171.704 108.763) (width 0.35) (layer F.Cu) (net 1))
 (segment (start 171.704 108.763) (end 170.485 108.763) (width 0.35) (layer F.Cu) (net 1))
 (segment (start 170.485 108.763) (end 169.977 108.255) (width 0.35) (layer F.Cu) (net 1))
 (segment (start 169.977 108.255) (end 169.977 106.426) (width 0.35) (layer F.Cu) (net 1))
 (segment (start 169.977 106.426) (end 168.808 105.258) (width 0.35) (layer F.Cu) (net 1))
 (segment (start 168.808 105.258) (end 167.691 105.258) (width 0.35) (layer F.Cu) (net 1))
 (segment (start 167.691 105.258) (end 166.472 104.038) (width 0.35) (layer F.Cu) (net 1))
 (segment (start 166.472 104.038) (end 166.472 101.752) (width 0.35) (layer F.Cu) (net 1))
 (segment (start 166.472 101.752) (end 163.728 99.0092) (width 0.35) (layer F.Cu) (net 1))
 (segment (start 163.728 99.0092) (end 163.728 97.0051) (width 0.35) (layer F.Cu) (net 1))
 (segment (start 168.91 110.998) (end 171.653 110.998) (width 0.35) (layer F.Cu) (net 1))
 (segment (start 163.728 97.0051) (end 164.132 97.0051) (width 0.35) (layer F.Cu) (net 1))
 (segment (start 164.132 97.0051) (end 166.049 95.0888) (width 0.35) (layer F.Cu) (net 1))
 (segment (start 166.049 95.0888) (end 168.749 95.0888) (width 0.35) (layer F.Cu) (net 1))
 (segment (start 168.749 95.0888) (end 169.062 95.4024) (width 0.35) (layer F.Cu) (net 1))
 (segment (start 169.062 95.4024) (end 169.062 98.6028) (width 0.35) (layer F.Cu) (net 1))
 (segment (start 169.062 98.6028) (end 169.367 98.9076) (width 0.35) (layer F.Cu) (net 1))
 (segment (start 169.367 98.9076) (end 172.441 98.9076) (width 0.35) (layer F.Cu) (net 1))
 (segment (start 172.441 98.9076) (end 172.872 98.4758) (width 0.35) (layer F.Cu) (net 1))
 (segment (start 172.872 98.4758) (end 172.872 97.0051) (width 0.35) (layer F.Cu) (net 1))
 (segment (start 158.826 115.849) (end 158.826 116.764) (width 0.35) (layer F.Cu) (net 1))
 (segment (start 158.826 115.849) (end 158.826 116.662) (width 0.35) (layer F.Cu) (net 1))
 (segment (start 158.826 116.662) (end 161.138 118.974) (width 0.35) (layer F.Cu) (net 1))
 (segment (start 161.138 118.974) (end 166.833 118.974) (width 0.35) (layer F.Cu) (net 1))
 (segment (start 166.833 118.974) (end 167.183 118.624) (width 0.35) (layer F.Cu) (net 1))
 (via (at 165.4842 112.6827) (size 0.6) (layers F.Cu B.Cu) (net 1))
 (segment (start 163.8295 106.553) (end 163.83 106.553) (width 0.35) (layer F.Cu) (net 7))
 (segment (start 163.906 115.849) (end 163.906 115.494) (width 0.35) (layer F.Cu) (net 7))
 (segment (start 163.906 115.494) (end 161.976 113.563) (width 0.35) (layer F.Cu) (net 7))
 (segment (start 161.976 113.563) (end 161.976 107.086) (width 0.35) (layer F.Cu) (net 7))
 (segment (start 161.976 107.086) (end 162.509 106.553) (width 0.35) (layer F.Cu) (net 7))
 (segment (start 162.509 106.553) (end 163.8295 106.553) (width 0.35) (layer F.Cu) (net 7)))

